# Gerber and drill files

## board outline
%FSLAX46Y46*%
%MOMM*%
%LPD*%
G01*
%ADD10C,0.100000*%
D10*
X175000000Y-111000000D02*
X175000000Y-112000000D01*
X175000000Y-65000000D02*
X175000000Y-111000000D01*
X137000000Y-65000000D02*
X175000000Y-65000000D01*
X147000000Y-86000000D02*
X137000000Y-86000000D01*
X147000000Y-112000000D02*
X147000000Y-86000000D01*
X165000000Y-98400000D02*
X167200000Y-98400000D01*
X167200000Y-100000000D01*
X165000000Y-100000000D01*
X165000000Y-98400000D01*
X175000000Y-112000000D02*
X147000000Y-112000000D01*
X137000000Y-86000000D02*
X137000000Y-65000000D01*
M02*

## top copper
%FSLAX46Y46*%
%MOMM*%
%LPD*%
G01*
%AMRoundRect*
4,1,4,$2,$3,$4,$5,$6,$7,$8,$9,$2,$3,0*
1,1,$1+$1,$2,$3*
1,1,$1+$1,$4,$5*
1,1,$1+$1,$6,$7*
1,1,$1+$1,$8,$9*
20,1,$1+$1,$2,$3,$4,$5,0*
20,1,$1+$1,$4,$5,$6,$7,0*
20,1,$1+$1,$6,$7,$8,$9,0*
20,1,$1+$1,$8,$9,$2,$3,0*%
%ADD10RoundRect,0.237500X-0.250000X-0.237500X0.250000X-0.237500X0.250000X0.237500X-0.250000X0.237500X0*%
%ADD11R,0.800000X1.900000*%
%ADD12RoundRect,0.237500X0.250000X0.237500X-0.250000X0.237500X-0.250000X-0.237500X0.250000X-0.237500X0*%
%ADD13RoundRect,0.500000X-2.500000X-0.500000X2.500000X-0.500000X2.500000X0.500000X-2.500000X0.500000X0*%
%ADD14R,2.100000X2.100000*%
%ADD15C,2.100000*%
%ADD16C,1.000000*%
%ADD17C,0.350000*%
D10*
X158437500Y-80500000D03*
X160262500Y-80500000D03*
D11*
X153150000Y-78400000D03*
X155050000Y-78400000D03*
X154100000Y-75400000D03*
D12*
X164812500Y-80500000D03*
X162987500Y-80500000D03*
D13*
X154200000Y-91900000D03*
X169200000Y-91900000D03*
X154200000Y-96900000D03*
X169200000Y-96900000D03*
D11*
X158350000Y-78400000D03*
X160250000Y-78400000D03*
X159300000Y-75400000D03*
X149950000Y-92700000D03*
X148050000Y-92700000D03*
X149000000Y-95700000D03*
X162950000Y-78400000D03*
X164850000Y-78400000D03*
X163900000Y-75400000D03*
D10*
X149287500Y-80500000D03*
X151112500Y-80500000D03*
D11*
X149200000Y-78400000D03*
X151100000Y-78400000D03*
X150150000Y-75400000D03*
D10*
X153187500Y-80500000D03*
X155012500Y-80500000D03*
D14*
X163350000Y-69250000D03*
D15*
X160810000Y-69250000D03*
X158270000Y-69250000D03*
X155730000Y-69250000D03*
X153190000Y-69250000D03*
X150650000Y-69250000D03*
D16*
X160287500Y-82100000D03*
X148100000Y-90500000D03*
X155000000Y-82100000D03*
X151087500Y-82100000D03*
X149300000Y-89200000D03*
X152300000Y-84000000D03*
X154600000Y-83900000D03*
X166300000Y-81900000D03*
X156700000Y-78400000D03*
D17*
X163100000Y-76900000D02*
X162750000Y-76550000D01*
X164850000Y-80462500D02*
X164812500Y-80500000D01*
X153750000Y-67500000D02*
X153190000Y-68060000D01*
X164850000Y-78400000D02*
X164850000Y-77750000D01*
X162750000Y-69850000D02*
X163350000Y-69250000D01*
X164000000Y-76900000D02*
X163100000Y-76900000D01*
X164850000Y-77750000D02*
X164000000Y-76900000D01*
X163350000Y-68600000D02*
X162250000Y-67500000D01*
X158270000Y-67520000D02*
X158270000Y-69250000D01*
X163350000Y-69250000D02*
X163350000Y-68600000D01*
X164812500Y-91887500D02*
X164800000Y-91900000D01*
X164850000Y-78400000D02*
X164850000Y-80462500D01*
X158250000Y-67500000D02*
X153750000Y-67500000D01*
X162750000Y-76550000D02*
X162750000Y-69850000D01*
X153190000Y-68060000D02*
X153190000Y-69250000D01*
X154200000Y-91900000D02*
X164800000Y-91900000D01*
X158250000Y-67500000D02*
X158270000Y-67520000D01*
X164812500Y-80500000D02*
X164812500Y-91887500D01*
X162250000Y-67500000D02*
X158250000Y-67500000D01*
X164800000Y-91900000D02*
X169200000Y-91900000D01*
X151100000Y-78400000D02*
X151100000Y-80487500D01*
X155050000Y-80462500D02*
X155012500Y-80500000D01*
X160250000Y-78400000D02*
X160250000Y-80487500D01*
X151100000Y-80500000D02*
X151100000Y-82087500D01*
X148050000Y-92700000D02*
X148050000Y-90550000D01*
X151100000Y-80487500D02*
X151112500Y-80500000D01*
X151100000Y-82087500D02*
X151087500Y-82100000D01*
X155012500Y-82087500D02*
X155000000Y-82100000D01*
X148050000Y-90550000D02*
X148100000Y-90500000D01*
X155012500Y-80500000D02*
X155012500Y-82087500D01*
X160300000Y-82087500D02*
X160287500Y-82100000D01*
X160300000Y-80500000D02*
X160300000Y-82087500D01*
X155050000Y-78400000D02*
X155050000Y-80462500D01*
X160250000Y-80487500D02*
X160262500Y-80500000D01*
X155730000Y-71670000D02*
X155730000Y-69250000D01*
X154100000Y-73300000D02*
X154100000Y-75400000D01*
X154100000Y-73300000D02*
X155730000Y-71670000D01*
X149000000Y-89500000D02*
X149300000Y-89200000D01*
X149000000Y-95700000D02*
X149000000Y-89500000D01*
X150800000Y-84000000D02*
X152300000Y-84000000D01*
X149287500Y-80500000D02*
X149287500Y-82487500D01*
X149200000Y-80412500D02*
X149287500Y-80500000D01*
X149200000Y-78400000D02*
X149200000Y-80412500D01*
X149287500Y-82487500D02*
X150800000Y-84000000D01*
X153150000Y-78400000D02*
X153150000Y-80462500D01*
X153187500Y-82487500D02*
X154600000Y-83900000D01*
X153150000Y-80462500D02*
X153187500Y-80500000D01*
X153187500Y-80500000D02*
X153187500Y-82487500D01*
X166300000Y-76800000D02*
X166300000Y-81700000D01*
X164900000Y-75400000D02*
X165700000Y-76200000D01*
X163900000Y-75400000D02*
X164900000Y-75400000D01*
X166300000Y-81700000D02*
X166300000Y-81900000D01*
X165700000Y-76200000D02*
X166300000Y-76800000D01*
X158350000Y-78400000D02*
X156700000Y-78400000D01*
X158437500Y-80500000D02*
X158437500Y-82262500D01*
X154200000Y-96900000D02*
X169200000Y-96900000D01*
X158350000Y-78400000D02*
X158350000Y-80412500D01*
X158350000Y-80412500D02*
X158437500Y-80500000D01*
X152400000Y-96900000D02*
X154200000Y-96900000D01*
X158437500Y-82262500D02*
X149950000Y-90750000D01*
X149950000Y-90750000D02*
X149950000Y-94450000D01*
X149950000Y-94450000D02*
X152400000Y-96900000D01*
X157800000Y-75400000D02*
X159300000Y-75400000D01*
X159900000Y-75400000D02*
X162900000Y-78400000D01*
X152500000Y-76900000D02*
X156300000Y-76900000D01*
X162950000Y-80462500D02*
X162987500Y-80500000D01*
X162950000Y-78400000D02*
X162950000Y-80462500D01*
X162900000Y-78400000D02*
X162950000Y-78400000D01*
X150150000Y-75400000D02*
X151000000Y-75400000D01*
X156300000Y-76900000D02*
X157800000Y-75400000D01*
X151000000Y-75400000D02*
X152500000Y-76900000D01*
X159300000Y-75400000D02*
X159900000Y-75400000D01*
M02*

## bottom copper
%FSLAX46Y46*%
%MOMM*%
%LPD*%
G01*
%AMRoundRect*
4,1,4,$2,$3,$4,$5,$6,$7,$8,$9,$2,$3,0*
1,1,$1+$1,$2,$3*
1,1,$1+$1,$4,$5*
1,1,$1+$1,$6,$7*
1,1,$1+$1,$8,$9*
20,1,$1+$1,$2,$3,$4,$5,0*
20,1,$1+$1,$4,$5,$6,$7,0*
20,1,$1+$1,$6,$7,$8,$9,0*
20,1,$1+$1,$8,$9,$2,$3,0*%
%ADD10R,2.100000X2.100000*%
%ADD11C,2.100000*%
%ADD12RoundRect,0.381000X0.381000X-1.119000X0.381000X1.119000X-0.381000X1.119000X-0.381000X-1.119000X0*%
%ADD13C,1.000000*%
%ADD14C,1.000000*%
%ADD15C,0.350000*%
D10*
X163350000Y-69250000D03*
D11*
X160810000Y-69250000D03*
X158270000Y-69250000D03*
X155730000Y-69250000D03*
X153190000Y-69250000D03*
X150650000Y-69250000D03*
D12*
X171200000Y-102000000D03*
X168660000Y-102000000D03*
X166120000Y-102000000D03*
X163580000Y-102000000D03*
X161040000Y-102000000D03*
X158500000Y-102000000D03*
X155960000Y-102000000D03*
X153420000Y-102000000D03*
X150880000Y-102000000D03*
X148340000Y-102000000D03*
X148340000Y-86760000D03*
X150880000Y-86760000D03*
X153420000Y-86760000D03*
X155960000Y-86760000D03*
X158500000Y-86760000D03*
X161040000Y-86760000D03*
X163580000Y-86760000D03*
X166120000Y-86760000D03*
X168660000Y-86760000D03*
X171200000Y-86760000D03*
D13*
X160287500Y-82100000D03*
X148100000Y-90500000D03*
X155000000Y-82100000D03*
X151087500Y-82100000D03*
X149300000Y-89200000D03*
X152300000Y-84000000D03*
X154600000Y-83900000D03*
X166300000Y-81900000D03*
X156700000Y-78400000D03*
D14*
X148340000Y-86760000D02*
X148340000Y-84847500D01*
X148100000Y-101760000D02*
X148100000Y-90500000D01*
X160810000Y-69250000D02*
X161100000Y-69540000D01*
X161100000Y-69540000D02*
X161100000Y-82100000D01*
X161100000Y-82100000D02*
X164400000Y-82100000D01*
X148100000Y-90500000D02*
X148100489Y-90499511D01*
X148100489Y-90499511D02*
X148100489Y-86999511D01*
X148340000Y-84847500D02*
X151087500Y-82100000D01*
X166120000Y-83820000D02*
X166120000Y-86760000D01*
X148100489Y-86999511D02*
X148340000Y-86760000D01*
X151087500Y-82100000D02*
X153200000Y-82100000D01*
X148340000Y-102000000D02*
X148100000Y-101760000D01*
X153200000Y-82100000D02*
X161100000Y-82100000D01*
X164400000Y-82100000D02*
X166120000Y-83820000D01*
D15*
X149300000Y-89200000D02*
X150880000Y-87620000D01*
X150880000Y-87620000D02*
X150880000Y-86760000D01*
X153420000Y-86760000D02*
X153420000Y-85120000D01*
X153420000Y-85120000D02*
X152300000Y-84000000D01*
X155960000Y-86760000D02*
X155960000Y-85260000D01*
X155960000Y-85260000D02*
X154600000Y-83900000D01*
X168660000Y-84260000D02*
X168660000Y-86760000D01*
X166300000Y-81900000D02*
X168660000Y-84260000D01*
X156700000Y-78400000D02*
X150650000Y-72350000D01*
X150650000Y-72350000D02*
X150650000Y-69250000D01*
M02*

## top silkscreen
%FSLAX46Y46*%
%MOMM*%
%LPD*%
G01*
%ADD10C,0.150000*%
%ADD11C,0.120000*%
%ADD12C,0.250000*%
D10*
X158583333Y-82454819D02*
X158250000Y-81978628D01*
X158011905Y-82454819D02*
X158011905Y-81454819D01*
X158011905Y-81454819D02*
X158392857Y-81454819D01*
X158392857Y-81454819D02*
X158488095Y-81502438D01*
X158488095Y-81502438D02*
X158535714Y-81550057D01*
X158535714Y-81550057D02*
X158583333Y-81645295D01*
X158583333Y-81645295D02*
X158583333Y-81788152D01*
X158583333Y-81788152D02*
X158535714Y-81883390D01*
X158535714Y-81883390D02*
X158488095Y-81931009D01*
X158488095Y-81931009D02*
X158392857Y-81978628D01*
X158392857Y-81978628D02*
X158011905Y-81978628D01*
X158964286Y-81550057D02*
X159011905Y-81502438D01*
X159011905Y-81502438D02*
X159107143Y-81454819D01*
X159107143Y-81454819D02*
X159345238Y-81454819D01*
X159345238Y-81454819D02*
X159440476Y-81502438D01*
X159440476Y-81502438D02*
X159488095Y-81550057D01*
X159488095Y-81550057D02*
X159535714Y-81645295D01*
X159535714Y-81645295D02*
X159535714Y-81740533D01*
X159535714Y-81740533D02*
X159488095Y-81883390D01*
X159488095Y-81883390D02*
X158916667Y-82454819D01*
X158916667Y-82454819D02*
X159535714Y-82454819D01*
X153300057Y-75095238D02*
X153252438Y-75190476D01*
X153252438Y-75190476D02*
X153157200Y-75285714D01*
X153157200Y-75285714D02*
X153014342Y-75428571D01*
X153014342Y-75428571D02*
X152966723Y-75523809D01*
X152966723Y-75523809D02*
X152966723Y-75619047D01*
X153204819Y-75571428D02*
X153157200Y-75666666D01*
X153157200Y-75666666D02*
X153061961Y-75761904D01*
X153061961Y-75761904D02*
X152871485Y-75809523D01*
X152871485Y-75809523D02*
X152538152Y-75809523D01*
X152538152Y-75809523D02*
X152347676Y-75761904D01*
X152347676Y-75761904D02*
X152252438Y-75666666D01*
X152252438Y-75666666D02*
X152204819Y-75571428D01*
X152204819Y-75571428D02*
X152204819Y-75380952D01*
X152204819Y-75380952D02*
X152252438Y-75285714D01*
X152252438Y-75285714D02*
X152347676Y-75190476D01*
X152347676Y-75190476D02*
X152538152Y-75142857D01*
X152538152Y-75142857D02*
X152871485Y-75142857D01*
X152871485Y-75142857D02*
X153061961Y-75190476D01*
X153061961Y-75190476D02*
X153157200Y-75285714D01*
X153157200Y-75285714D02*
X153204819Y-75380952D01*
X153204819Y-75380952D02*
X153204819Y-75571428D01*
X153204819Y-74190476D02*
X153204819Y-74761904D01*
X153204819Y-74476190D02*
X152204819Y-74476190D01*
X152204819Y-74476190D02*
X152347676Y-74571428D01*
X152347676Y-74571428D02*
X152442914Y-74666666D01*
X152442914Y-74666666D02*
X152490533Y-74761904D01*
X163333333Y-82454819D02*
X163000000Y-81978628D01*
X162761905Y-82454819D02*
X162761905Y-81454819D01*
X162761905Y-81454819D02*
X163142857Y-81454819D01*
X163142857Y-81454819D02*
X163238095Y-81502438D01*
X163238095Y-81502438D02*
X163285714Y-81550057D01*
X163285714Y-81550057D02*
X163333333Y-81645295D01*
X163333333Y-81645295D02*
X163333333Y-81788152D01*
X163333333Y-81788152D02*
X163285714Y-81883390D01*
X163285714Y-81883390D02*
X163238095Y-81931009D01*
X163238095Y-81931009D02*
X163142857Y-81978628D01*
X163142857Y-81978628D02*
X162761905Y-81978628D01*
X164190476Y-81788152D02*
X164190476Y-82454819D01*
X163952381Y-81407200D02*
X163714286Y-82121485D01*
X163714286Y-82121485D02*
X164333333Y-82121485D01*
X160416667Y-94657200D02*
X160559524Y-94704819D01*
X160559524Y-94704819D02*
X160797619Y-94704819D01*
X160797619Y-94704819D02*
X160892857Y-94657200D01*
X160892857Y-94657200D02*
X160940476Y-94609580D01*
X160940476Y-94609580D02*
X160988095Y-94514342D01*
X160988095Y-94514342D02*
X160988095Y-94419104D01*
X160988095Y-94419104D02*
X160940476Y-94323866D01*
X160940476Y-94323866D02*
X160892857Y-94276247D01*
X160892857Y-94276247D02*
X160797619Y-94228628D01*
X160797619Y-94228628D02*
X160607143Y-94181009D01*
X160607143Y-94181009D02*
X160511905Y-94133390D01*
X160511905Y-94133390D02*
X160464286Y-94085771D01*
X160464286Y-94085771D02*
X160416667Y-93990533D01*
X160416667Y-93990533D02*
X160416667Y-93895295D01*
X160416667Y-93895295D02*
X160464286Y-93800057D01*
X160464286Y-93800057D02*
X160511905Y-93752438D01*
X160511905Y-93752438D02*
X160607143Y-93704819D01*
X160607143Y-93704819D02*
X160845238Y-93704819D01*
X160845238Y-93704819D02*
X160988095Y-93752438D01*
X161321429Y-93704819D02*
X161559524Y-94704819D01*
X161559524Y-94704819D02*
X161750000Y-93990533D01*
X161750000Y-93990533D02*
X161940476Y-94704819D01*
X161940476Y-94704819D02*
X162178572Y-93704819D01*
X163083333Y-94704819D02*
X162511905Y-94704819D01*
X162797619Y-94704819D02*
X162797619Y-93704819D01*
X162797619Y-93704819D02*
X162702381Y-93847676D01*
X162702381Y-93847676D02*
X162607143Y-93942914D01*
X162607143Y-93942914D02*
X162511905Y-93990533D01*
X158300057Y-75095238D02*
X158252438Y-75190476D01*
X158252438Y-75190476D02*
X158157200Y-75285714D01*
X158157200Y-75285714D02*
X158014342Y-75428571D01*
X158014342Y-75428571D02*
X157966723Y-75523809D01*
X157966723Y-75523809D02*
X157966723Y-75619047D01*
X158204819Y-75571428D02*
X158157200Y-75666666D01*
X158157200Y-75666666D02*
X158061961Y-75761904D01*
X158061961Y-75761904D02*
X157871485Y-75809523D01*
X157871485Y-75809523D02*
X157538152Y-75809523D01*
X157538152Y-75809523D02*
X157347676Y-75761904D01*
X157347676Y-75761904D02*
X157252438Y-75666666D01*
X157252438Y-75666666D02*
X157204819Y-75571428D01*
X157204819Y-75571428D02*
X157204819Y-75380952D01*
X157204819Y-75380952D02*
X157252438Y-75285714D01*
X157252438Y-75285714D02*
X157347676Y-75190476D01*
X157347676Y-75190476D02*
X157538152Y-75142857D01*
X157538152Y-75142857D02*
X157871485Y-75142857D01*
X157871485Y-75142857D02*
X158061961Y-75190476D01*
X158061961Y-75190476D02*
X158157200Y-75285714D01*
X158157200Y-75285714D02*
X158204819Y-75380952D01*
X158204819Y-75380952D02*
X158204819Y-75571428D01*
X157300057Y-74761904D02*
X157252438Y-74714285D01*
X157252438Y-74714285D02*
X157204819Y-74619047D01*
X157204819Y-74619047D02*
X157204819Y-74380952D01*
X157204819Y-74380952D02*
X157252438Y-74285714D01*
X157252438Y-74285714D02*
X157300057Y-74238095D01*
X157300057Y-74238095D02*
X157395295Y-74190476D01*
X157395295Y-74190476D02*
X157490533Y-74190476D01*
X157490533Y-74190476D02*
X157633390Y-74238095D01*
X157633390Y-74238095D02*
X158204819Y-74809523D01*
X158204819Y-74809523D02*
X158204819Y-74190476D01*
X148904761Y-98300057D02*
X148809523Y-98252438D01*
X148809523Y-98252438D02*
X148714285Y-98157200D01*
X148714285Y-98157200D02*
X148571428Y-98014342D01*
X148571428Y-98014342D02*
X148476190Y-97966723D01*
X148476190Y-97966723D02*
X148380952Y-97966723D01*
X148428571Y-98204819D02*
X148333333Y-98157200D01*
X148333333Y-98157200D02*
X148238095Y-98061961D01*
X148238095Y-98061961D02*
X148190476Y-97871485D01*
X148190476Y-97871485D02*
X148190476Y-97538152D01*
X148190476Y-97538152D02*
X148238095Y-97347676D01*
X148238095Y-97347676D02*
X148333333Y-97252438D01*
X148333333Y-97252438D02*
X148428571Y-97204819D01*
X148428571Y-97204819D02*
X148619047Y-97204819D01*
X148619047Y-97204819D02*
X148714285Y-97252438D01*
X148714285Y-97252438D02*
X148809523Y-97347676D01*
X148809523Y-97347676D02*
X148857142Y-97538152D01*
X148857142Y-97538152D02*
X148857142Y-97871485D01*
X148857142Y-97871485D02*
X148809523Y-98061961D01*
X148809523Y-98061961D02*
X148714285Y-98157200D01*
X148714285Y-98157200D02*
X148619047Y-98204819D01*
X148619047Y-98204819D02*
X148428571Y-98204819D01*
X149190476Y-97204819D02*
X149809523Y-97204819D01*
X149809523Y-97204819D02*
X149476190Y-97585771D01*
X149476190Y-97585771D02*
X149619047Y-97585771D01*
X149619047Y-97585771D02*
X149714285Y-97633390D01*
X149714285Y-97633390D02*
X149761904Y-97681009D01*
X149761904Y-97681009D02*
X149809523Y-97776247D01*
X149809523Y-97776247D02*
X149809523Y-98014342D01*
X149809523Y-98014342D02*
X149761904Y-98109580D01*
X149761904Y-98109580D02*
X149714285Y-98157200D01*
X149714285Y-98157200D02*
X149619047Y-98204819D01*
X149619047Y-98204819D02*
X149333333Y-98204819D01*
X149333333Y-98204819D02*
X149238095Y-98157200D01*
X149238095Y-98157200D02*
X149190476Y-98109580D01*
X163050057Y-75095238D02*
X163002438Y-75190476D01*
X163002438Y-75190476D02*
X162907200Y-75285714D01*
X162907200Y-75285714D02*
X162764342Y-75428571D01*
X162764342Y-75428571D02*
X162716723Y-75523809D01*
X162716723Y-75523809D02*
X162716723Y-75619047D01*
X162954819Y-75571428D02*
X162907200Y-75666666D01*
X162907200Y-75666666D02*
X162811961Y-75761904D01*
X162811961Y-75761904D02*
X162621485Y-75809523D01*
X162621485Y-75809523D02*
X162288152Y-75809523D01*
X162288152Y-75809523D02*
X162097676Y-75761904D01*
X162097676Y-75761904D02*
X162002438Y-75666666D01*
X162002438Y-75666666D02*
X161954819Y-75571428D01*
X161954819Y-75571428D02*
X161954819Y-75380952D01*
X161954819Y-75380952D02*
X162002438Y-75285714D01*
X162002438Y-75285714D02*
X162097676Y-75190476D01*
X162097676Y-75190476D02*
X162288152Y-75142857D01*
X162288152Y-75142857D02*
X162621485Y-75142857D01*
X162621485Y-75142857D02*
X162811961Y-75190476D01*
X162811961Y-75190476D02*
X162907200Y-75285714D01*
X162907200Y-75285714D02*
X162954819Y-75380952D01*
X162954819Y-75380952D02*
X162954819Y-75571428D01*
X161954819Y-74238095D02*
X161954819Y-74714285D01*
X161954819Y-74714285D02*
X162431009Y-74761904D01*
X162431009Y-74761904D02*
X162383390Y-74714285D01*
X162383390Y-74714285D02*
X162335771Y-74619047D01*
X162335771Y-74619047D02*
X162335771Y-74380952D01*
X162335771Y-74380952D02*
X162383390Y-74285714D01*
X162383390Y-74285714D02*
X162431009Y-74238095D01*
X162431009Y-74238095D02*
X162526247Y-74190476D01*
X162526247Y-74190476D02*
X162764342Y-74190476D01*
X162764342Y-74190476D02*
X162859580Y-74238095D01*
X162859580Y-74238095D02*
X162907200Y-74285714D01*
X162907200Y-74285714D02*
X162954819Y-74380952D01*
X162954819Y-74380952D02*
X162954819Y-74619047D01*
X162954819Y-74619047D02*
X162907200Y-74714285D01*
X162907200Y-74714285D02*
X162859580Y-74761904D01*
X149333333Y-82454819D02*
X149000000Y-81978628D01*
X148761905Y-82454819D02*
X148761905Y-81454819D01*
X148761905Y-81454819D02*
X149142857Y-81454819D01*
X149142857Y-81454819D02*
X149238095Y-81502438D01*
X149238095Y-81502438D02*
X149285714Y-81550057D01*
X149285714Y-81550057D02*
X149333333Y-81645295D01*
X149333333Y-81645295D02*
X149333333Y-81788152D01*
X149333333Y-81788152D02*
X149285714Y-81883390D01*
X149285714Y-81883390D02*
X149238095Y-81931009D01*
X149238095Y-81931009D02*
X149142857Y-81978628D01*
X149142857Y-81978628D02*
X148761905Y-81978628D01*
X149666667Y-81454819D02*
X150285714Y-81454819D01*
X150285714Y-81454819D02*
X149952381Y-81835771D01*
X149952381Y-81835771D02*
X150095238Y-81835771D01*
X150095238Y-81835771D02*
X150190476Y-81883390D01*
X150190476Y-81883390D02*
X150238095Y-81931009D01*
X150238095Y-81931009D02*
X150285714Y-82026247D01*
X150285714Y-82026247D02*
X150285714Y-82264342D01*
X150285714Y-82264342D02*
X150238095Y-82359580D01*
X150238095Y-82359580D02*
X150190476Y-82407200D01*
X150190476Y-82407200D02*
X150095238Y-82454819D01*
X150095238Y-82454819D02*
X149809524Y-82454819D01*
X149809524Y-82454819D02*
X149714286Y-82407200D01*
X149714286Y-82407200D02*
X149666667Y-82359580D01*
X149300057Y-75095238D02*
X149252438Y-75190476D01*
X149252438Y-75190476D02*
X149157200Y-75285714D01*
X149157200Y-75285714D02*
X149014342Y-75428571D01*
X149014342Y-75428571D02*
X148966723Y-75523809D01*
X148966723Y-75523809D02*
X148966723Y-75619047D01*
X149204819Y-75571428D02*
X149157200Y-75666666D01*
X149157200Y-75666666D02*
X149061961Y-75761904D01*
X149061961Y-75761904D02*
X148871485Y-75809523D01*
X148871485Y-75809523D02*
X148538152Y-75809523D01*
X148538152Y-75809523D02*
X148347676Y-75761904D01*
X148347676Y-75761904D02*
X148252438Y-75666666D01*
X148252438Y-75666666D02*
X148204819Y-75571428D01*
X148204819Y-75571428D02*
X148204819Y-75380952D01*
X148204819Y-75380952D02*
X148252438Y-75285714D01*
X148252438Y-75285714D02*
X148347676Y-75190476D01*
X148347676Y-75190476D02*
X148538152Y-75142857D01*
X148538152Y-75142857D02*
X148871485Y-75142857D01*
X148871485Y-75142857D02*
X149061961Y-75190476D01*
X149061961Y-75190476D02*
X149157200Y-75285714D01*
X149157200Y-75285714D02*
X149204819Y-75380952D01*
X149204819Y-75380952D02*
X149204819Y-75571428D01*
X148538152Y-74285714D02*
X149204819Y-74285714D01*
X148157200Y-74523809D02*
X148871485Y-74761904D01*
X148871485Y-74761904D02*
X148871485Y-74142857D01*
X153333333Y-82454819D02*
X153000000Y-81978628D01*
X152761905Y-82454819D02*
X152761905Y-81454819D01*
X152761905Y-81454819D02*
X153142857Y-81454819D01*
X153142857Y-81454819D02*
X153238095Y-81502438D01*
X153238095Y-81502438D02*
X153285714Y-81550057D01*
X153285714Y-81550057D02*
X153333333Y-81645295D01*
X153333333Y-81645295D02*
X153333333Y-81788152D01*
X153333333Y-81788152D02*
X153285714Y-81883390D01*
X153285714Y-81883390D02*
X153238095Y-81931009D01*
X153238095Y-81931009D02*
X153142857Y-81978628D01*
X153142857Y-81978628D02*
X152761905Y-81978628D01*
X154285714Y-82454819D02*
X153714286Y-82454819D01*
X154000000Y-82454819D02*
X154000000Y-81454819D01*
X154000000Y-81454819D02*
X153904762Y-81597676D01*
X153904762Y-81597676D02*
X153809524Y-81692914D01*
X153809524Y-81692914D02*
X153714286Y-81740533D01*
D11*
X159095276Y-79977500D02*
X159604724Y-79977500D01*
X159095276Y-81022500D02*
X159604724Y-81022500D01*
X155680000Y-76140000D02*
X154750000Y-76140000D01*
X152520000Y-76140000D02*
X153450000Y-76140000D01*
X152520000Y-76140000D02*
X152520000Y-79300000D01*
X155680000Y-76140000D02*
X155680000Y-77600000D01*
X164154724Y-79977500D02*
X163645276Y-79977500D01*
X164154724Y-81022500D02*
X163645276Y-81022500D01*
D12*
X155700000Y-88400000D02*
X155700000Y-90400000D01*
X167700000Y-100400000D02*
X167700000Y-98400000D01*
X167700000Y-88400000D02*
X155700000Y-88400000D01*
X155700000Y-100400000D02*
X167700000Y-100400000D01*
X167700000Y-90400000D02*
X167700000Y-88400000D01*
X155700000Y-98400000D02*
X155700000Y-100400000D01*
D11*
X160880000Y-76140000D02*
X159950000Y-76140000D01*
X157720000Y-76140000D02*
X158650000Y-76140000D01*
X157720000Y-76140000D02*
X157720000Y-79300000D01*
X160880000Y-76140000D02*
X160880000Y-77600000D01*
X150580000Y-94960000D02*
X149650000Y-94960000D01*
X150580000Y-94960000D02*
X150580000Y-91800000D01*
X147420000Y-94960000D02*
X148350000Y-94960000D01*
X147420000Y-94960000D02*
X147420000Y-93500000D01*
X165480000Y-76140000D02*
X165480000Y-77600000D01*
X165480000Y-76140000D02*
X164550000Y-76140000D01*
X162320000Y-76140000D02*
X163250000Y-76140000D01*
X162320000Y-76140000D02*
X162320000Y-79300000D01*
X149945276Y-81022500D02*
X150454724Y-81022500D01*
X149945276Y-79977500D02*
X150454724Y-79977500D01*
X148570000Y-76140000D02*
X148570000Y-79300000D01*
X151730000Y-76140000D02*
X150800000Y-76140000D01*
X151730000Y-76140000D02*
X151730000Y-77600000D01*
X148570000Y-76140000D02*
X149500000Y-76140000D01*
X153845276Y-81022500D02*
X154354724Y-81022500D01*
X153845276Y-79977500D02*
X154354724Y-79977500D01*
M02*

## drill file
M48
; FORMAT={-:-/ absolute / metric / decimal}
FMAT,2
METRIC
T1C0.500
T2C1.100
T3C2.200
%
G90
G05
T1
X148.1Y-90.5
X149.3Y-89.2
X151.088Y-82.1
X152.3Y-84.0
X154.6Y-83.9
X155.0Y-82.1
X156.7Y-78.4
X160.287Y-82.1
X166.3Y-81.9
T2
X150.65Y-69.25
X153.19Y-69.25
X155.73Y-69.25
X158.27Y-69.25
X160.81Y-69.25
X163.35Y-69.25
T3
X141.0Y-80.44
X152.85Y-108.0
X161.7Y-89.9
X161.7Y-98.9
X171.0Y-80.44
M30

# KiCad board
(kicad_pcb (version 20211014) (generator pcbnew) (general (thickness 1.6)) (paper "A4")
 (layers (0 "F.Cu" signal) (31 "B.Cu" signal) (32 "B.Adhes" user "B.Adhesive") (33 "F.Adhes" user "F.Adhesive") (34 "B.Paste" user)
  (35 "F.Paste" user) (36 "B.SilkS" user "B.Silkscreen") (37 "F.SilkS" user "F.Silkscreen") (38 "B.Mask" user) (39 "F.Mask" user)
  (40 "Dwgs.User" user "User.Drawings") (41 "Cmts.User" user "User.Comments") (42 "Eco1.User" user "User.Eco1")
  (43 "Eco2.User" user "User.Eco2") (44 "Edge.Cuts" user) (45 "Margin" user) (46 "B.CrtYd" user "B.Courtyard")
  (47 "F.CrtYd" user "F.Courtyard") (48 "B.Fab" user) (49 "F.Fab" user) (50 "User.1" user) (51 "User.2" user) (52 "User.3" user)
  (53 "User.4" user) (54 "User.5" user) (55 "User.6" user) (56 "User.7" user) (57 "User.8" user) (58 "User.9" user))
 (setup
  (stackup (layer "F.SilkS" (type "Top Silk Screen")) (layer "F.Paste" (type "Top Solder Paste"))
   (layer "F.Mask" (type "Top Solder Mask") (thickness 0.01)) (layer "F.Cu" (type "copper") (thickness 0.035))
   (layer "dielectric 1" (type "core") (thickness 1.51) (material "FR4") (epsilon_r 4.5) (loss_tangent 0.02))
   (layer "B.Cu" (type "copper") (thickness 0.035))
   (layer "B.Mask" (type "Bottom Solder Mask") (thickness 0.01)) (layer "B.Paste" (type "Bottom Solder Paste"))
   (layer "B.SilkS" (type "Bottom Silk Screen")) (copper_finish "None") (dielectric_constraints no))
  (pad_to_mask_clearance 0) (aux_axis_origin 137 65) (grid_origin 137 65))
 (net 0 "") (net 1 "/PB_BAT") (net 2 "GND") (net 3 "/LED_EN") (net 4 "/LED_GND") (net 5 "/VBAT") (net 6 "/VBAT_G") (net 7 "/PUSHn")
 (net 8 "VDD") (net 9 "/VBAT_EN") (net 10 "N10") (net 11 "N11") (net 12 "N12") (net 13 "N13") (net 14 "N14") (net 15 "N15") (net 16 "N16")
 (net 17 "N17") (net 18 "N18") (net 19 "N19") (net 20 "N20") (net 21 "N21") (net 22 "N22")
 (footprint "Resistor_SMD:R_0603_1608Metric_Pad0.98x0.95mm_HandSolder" (layer "F.Cu") (at 159.35 80.5)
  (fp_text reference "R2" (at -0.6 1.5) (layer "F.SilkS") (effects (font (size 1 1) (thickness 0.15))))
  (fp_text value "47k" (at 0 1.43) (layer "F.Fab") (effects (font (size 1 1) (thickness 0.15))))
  (fp_line (start -0.254724 -0.5225) (end 0.254724 -0.5225) (layer "F.SilkS") (width 0.12))
  (fp_line (start -0.254724 0.5225) (end 0.254724 0.5225) (layer "F.SilkS") (width 0.12))
  (pad "1" smd roundrect (at -0.9125 0) (size 0.975 0.95) (layers "F.Cu" "F.Paste" "F.Mask") (roundrect_rratio 0.25) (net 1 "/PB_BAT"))
  (pad "2" smd roundrect (at 0.9125 0) (size 0.975 0.95) (layers "F.Cu" "F.Paste" "F.Mask") (roundrect_rratio 0.25) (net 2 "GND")))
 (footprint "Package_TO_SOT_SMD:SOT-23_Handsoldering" (layer "F.Cu") (at 154.1 76.9 90)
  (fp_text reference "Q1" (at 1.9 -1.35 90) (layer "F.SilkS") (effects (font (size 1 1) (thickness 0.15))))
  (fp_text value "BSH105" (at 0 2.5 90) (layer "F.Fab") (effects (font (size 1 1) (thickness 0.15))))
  (fp_line (start 0.76 1.58) (end 0.76 0.65) (layer "F.SilkS") (width 0.12))
  (fp_line (start 0.76 -1.58) (end 0.76 -0.65) (layer "F.SilkS") (width 0.12))
  (fp_line (start 0.76 -1.58) (end -2.4 -1.58) (layer "F.SilkS") (width 0.12))
  (fp_line (start 0.76 1.58) (end -0.7 1.58) (layer "F.SilkS") (width 0.12))
  (pad "1" smd rect (at -1.5 -0.95 90) (size 1.9 0.8) (layers "F.Cu" "F.Paste" "F.Mask") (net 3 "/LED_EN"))
  (pad "2" smd rect (at -1.5 0.95 90) (size 1.9 0.8) (layers "F.Cu" "F.Paste" "F.Mask") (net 2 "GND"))
  (pad "3" smd rect (at 1.5 0 90) (size 1.9 0.8) (layers "F.Cu" "F.Paste" "F.Mask") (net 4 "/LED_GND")))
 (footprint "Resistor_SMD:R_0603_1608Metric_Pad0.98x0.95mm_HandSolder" (layer "F.Cu") (at 163.9 80.5 180)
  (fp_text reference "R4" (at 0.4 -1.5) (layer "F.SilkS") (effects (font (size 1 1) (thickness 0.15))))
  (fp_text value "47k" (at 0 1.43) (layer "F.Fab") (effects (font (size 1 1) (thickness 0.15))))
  (fp_line (start -0.254724 0.5225) (end 0.254724 0.5225) (layer "F.SilkS") (width 0.12))
  (fp_line (start -0.254724 -0.5225) (end 0.254724 -0.5225) (layer "F.SilkS") (width 0.12))
  (pad "1" smd roundrect (at -0.9125 0 180) (size 0.975 0.95) (layers "F.Cu" "F.Paste" "F.Mask") (roundrect_rratio 0.25) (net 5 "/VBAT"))
  (pad "2" smd roundrect (at 0.9125 0 180) (size 0.975 0.95) (layers "F.Cu" "F.Paste" "F.Mask") (roundrect_rratio 0.25) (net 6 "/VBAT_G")))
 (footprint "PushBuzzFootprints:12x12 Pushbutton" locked (layer "F.Cu") (at 154.2 91.9)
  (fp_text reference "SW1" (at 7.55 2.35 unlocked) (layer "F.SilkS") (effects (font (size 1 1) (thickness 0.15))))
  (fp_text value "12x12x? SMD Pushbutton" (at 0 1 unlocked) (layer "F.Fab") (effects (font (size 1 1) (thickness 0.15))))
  (fp_line (start 1.5 -3.5) (end 1.5 -1.5) (layer "F.SilkS") (width 0.25))
  (fp_line (start 13.5 8.5) (end 13.5 6.5) (layer "F.SilkS") (width 0.25))
  (fp_line (start 13.5 -3.5) (end 1.5 -3.5) (layer "F.SilkS") (width 0.25))
  (fp_line (start 1.5 8.5) (end 13.5 8.5) (layer "F.SilkS") (width 0.25))
  (fp_line (start 13.5 -1.5) (end 13.5 -3.5) (layer "F.SilkS") (width 0.25))
  (fp_line (start 1.5 6.5) (end 1.5 8.5) (layer "F.SilkS") (width 0.25))
  (pad "" np_thru_hole circle locked (at 7.5 -2) (size 2 2) (drill 2.2) (layers F&B.Cu *.Mask))
  (pad "" np_thru_hole circle locked (at 7.5 7) (size 2 2) (drill 2.2) (layers F&B.Cu *.Mask))
  (pad "1" smd roundrect locked (at 0 0) (size 6 2) (layers "F.Cu" "F.Paste" "F.Mask") (roundrect_rratio 0.25) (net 5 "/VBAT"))
  (pad "1" smd roundrect locked (at 15 0) (size 6 2) (layers "F.Cu" "F.Paste" "F.Mask") (roundrect_rratio 0.25) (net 5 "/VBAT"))
  (pad "2" smd roundrect locked (at 0 5) (size 6 2) (layers "F.Cu" "F.Paste" "F.Mask") (roundrect_rratio 0.25) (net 1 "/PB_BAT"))
  (pad "2" smd roundrect locked (at 15 5) (size 6 2) (layers "F.Cu" "F.Paste" "F.Mask") (roundrect_rratio 0.25) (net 1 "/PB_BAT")))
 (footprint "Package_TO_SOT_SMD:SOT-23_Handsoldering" (layer "F.Cu") (at 159.3 76.9 90)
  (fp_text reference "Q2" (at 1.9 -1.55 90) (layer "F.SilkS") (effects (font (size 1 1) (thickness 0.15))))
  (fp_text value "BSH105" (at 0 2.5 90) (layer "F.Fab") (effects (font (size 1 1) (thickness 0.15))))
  (fp_line (start 0.76 1.58) (end 0.76 0.65) (layer "F.SilkS") (width 0.12))
  (fp_line (start 0.76 -1.58) (end 0.76 -0.65) (layer "F.SilkS") (width 0.12))
  (fp_line (start 0.76 -1.58) (end -2.4 -1.58) (layer "F.SilkS") (width 0.12))
  (fp_line (start 0.76 1.58) (end -0.7 1.58) (layer "F.SilkS") (width 0.12))
  (pad "1" smd rect (at -1.5 -0.95 90) (size 1.9 0.8) (layers "F.Cu" "F.Paste" "F.Mask") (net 1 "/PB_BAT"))
  (pad "2" smd rect (at -1.5 0.95 90) (size 1.9 0.8) (layers "F.Cu" "F.Paste" "F.Mask") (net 2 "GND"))
  (pad "3" smd rect (at 1.5 0 90) (size 1.9 0.8) (layers "F.Cu" "F.Paste" "F.Mask") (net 6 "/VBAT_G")))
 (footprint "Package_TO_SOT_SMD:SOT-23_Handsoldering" (layer "F.Cu") (at 149 94.2 -90)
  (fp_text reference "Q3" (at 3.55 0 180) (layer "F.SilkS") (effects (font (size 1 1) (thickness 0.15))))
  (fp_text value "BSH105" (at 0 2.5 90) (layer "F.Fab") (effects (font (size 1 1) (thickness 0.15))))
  (fp_line (start 0.76 -1.58) (end 0.76 -0.65) (layer "F.SilkS") (width 0.12))
  (fp_line (start 0.76 -1.58) (end -2.4 -1.58) (layer "F.SilkS") (width 0.12))
  (fp_line (start 0.76 1.58) (end 0.76 0.65) (layer "F.SilkS") (width 0.12))
  (fp_line (start 0.76 1.58) (end -0.7 1.58) (layer "F.SilkS") (width 0.12))
  (pad "1" smd rect (at -1.5 -0.95 270) (size 1.9 0.8) (layers "F.Cu" "F.Paste" "F.Mask") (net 1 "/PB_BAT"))
  (pad "2" smd rect (at -1.5 0.95 270) (size 1.9 0.8) (layers "F.Cu" "F.Paste" "F.Mask") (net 2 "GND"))
  (pad "3" smd rect (at 1.5 0 270) (size 1.9 0.8) (layers "F.Cu" "F.Paste" "F.Mask") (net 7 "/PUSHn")))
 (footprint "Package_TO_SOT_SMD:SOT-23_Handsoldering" (layer "F.Cu") (at 163.9 76.9 90)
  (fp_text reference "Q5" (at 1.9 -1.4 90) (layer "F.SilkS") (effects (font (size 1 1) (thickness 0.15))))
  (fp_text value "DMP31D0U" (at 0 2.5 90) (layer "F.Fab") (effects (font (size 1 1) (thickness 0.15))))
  (fp_line (start 0.76 1.58) (end -0.7 1.58) (layer "F.SilkS") (width 0.12))
  (fp_line (start 0.76 1.58) (end 0.76 0.65) (layer "F.SilkS") (width 0.12))
  (fp_line (start 0.76 -1.58) (end 0.76 -0.65) (layer "F.SilkS") (width 0.12))
  (fp_line (start 0.76 -1.58) (end -2.4 -1.58) (layer "F.SilkS") (width 0.12))
  (pad "1" smd rect (at -1.5 -0.95 90) (size 1.9 0.8) (layers "F.Cu" "F.Paste" "F.Mask") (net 6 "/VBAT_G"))
  (pad "2" smd rect (at -1.5 0.95 90) (size 1.9 0.8) (layers "F.Cu" "F.Paste" "F.Mask") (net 5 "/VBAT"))
  (pad "3" smd rect (at 1.5 0 90) (size 1.9 0.8) (layers "F.Cu" "F.Paste" "F.Mask") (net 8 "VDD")))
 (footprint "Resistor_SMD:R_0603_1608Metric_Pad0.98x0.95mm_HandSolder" (layer "F.Cu") (at 150.2 80.5)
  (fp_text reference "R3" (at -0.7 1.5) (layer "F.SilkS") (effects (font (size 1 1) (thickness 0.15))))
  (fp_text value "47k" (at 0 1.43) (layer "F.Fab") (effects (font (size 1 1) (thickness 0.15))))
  (fp_line (start -0.254724 0.5225) (end 0.254724 0.5225) (layer "F.SilkS") (width 0.12))
  (fp_line (start -0.254724 -0.5225) (end 0.254724 -0.5225) (layer "F.SilkS") (width 0.12))
  (pad "1" smd roundrect (at -0.9125 0) (size 0.975 0.95) (layers "F.Cu" "F.Paste" "F.Mask") (roundrect_rratio 0.25) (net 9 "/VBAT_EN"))
  (pad "2" smd roundrect (at 0.9125 0) (size 0.975 0.95) (layers "F.Cu" "F.Paste" "F.Mask") (roundrect_rratio 0.25) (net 2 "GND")))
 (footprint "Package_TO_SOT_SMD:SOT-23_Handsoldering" (layer "F.Cu") (at 150.15 76.9 90)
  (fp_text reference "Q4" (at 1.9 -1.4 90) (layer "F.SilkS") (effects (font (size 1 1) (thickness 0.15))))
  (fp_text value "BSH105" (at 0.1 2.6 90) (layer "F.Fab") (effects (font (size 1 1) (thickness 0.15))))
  (fp_line (start 0.76 -1.58) (end -2.4 -1.58) (layer "F.SilkS") (width 0.12))
  (fp_line (start 0.76 1.58) (end 0.76 0.65) (layer "F.SilkS") (width 0.12))
  (fp_line (start 0.76 1.58) (end -0.7 1.58) (layer "F.SilkS") (width 0.12))
  (fp_line (start 0.76 -1.58) (end 0.76 -0.65) (layer "F.SilkS") (width 0.12))
  (pad "1" smd rect (at -1.5 -0.95 90) (size 1.9 0.8) (layers "F.Cu" "F.Paste" "F.Mask") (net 9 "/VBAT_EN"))
  (pad "2" smd rect (at -1.5 0.95 90) (size 1.9 0.8) (layers "F.Cu" "F.Paste" "F.Mask") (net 2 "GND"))
  (pad "3" smd rect (at 1.5 0 90) (size 1.9 0.8) (layers "F.Cu" "F.Paste" "F.Mask") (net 6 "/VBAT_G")))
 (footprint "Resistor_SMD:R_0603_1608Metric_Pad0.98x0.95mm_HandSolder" (layer "F.Cu") (at 154.1 80.5)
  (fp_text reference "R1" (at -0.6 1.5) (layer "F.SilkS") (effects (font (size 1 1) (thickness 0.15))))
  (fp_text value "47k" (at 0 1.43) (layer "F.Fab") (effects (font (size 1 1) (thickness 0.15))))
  (fp_line (start -0.254724 0.5225) (end 0.254724 0.5225) (layer "F.SilkS") (width 0.12))
  (fp_line (start -0.254724 -0.5225) (end 0.254724 -0.5225) (layer "F.SilkS") (width 0.12))
  (pad "1" smd roundrect (at -0.9125 0) (size 0.975 0.95) (layers "F.Cu" "F.Paste" "F.Mask") (roundrect_rratio 0.25) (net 3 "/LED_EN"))
  (pad "2" smd roundrect (at 0.9125 0) (size 0.975 0.95) (layers "F.Cu" "F.Paste" "F.Mask") (roundrect_rratio 0.25) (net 2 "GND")))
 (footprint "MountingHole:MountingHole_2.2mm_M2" (layer "B.Cu") (at 152.85 108 180)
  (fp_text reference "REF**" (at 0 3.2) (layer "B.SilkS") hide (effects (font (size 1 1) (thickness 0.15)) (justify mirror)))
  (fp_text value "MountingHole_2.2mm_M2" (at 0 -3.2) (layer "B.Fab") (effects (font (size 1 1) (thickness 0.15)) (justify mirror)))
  (pad "" np_thru_hole circle (at 0 0 180) (size 2.2 2.2) (drill 2.2) (layers *.Cu *.Mask)))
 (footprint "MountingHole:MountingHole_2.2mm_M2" (layer "B.Cu") (at 141 80.44 180)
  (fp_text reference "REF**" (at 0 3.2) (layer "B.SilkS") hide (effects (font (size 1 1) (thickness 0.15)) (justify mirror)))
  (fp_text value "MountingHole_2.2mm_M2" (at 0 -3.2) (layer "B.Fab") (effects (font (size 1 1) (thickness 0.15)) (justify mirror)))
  (pad "" np_thru_hole circle (at 0 0 180) (size 2.2 2.2) (drill 2.2) (layers *.Cu *.Mask)))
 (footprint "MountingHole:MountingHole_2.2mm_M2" (layer "B.Cu") (at 171 80.44 180)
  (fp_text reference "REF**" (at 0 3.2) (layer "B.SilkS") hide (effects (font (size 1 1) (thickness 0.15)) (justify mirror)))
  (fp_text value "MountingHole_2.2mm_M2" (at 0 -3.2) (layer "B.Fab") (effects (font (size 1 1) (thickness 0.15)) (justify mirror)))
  (pad "" np_thru_hole circle (at 0 0 180) (size 2.2 2.2) (drill 2.2) (layers *.Cu *.Mask)))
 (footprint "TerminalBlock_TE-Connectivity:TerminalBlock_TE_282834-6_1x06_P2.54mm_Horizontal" (layer "B.Cu") (at 163.35 69.25 180)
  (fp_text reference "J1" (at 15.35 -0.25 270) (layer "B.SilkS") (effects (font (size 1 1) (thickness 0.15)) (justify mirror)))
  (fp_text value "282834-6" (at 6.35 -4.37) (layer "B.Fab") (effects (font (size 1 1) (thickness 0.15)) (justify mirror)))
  (pad "1" thru_hole rect (at 0 0 180) (size 2.1 2.1) (drill 1.1) (layers *.Cu *.Mask) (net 5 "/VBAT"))
  (pad "2" thru_hole circle (at 2.54 0 180) (size 2.1 2.1) (drill 1.1) (layers *.Cu *.Mask) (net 2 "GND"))
  (pad "3" thru_hole circle (at 5.08 0 180) (size 2.1 2.1) (drill 1.1) (layers *.Cu *.Mask) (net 5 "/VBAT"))
  (pad "4" thru_hole circle (at 7.62 0 180) (size 2.1 2.1) (drill 1.1) (layers *.Cu *.Mask) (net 4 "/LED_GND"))
  (pad "5" thru_hole circle (at 10.16 0 180) (size 2.1 2.1) (drill 1.1) (layers *.Cu *.Mask) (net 5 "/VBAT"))
  (pad "6" thru_hole circle (at 12.7 0 180) (size 2.1 2.1) (drill 1.1) (layers *.Cu *.Mask) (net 1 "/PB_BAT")))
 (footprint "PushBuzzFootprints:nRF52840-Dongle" (layer "B.Cu") (at 171.2 102 90)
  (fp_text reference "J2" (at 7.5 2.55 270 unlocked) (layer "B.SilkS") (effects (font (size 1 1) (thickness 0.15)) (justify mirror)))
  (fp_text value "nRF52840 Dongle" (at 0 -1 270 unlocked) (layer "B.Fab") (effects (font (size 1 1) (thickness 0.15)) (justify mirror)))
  (pad "1" smd roundrect (at 0 0 90) (size 3 1.524) (layers "B.Cu" "B.Paste" "B.Mask") (roundrect_rratio 0.25) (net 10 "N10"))
  (pad "2" smd roundrect (at 0 -2.54 90) (size 3 1.524) (layers "B.Cu" "B.Paste" "B.Mask") (roundrect_rratio 0.25) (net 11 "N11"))
  (pad "3" smd roundrect (at 0 -5.08 90) (size 3 1.524) (layers "B.Cu" "B.Paste" "B.Mask") (roundrect_rratio 0.25) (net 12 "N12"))
  (pad "4" smd roundrect (at 0 -7.62 90) (size 3 1.524) (layers "B.Cu" "B.Paste" "B.Mask") (roundrect_rratio 0.25) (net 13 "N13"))
  (pad "5" smd roundrect (at 0 -10.16 90) (size 3 1.524) (layers "B.Cu" "B.Paste" "B.Mask") (roundrect_rratio 0.25) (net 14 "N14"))
  (pad "6" smd roundrect (at 0 -12.7 90) (size 3 1.524) (layers "B.Cu" "B.Paste" "B.Mask") (roundrect_rratio 0.25) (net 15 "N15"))
  (pad "7" smd roundrect (at 0 -15.24 90) (size 3 1.524) (layers "B.Cu" "B.Paste" "B.Mask") (roundrect_rratio 0.25) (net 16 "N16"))
  (pad "8" smd roundrect (at 0 -17.78 90) (size 3 1.524) (layers "B.Cu" "B.Paste" "B.Mask") (roundrect_rratio 0.25) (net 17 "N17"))
  (pad "9" smd roundrect (at 0 -20.32 90) (size 3 1.524) (layers "B.Cu" "B.Paste" "B.Mask") (roundrect_rratio 0.25) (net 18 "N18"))
  (pad "10" smd roundrect (at 0 -22.86 90) (size 3 1.524) (layers "B.Cu" "B.Paste" "B.Mask") (roundrect_rratio 0.25) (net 2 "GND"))
  (pad "11" smd roundrect (at 15.24 -22.86 90) (size 3 1.524) (layers "B.Cu" "B.Paste" "B.Mask") (roundrect_rratio 0.25) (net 2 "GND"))
  (pad "12" smd roundrect (at 15.24 -20.32 90) (size 3 1.524) (layers "B.Cu" "B.Paste" "B.Mask") (roundrect_rratio 0.25) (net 7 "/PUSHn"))
  (pad "13" smd roundrect (at 15.24 -17.78 90) (size 3 1.524) (layers "B.Cu" "B.Paste" "B.Mask") (roundrect_rratio 0.25) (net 9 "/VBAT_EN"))
  (pad "14" smd roundrect (at 15.24 -15.24 90) (size 3 1.524) (layers "B.Cu" "B.Paste" "B.Mask") (roundrect_rratio 0.25) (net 3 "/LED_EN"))
  (pad "15" smd roundrect (at 15.24 -12.7 90) (size 3 1.524) (layers "B.Cu" "B.Paste" "B.Mask") (roundrect_rratio 0.25) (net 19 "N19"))
  (pad "16" smd roundrect (at 15.24 -10.16 90) (size 3 1.524) (layers "B.Cu" "B.Paste" "B.Mask") (roundrect_rratio 0.25) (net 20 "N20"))
  (pad "17" smd roundrect (at 15.24 -7.62 90) (size 3 1.524) (layers "B.Cu" "B.Paste" "B.Mask") (roundrect_rratio 0.25) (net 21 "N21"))
  (pad "18" smd roundrect (at 15.24 -5.08 90) (size 3 1.524) (layers "B.Cu" "B.Paste" "B.Mask") (roundrect_rratio 0.25) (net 2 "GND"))
  (pad "19" smd roundrect (at 15.24 -2.54 90) (size 3 1.524) (layers "B.Cu" "B.Paste" "B.Mask") (roundrect_rratio 0.25) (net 8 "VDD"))
  (pad "20" smd roundrect (at 15.24 0 90) (size 3 1.524) (layers "B.Cu" "B.Paste" "B.Mask") (roundrect_rratio 0.25) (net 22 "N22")))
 (gr_line (start 175 111) (end 175 112) (layer "Edge.Cuts") (width 0.1))
 (gr_line (start 175 65) (end 175 111) (layer "Edge.Cuts") (width 0.1))
 (gr_line (start 137 65) (end 175 65) (layer "Edge.Cuts") (width 0.1))
 (gr_line (start 147 86) (end 137 86) (layer "Edge.Cuts") (width 0.1))
 (gr_line (start 147 112) (end 147 86) (layer "Edge.Cuts") (width 0.1))
 (gr_rect locked (start 165 100) (end 167.2 98.4) (layer "Edge.Cuts") (width 0.1) (fill none))
 (gr_line (start 175 112) (end 147 112) (layer "Edge.Cuts") (width 0.1))
 (gr_line (start 137 86) (end 137 65) (layer "Edge.Cuts") (width 0.1))
 (segment (start 163.1 76.9) (end 162.75 76.55) (width 0.35) (layer "F.Cu") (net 5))
 (segment (start 164.85 80.4625) (end 164.8125 80.5) (width 0.35) (layer "F.Cu") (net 5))
 (segment (start 153.75 67.5) (end 153.19 68.06) (width 0.35) (layer "F.Cu") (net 5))
 (segment (start 164.85 78.4) (end 164.85 77.75) (width 0.35) (layer "F.Cu") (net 5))
 (segment (start 162.75 69.85) (end 163.35 69.25) (width 0.35) (layer "F.Cu") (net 5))
 (segment (start 164 76.9) (end 163.1 76.9) (width 0.35) (layer "F.Cu") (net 5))
 (segment (start 164.85 77.75) (end 164 76.9) (width 0.35) (layer "F.Cu") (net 5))
 (segment (start 163.35 68.6) (end 162.25 67.5) (width 0.35) (layer "F.Cu") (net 5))
 (segment (start 158.27 67.52) (end 158.27 69.25) (width 0.35) (layer "F.Cu") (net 5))
 (segment (start 163.35 69.25) (end 163.35 68.6) (width 0.35) (layer "F.Cu") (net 5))
 (segment (start 164.8125 91.8875) (end 164.8 91.9) (width 0.35) (layer "F.Cu") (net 5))
 (segment (start 164.85 78.4) (end 164.85 80.4625) (width 0.35) (layer "F.Cu") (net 5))
 (segment (start 158.25 67.5) (end 153.75 67.5) (width 0.35) (layer "F.Cu") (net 5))
 (segment (start 162.75 76.55) (end 162.75 69.85) (width 0.35) (layer "F.Cu") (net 5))
 (segment (start 153.19 68.06) (end 153.19 69.25) (width 0.35) (layer "F.Cu") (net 5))
 (segment (start 154.2 91.9) (end 164.8 91.9) (width 0.35) (layer "F.Cu") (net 5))
 (segment (start 158.25 67.5) (end 158.27 67.52) (width 0.35) (layer "F.Cu") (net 5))
 (segment (start 164.8125 80.5) (end 164.8125 91.8875) (width 0.35) (layer "F.Cu") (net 5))
 (segment (start 162.25 67.5) (end 158.25 67.5) (width 0.35) (layer "F.Cu") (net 5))
 (segment (start 164.8 91.9) (end 169.2 91.9) (width 0.35) (layer "F.Cu") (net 5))
 (segment (start 151.1 78.4) (end 151.1 80.4875) (width 0.35) (layer "F.Cu") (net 2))
 (segment (start 155.05 80.4625) (end 155.0125 80.5) (width 0.35) (layer "F.Cu") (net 2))
 (segment (start 160.25 78.4) (end 160.25 80.4875) (width 0.35) (layer "F.Cu") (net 2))
 (segment (start 151.1 80.5) (end 151.1 82.0875) (width 0.35) (layer "F.Cu") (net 2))
 (segment (start 148.05 92.7) (end 148.05 90.55) (width 0.35) (layer "F.Cu") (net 2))
 (segment (start 151.1 80.4875) (end 151.1125 80.5) (width 0.35) (layer "F.Cu") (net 2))
 (segment (start 151.1 82.0875) (end 151.0875 82.1) (width 0.35) (layer "F.Cu") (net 2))
 (segment (start 155.0125 82.0875) (end 155 82.1) (width 0.35) (layer "F.Cu") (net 2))
 (segment (start 148.05 90.55) (end 148.1 90.5) (width 0.35) (layer "F.Cu") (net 2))
 (segment (start 155.0125 80.5) (end 155.0125 82.0875) (width 0.35) (layer "F.Cu") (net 2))
 (segment (start 160.3 82.0875) (end 160.2875 82.1) (width 0.35) (layer "F.Cu") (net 2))
 (segment (start 160.3 80.5) (end 160.3 82.0875) (width 0.35) (layer "F.Cu") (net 2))
 (segment (start 155.05 78.4) (end 155.05 80.4625) (width 0.35) (layer "F.Cu") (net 2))
 (segment (start 160.25 80.4875) (end 160.2625 80.5) (width 0.35) (layer "F.Cu") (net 2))
 (via (at 160.2875 82.1) (size 1) (drill 0.5) (layers "F.Cu" "B.Cu") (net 2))
 (via (at 148.1 90.5) (size 1) (drill 0.5) (layers "F.Cu" "B.Cu") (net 2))
 (via (at 155 82.1) (size 1) (drill 0.5) (layers "F.Cu" "B.Cu") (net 2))
 (via (at 151.0875 82.1) (size 1) (drill 0.5) (layers "F.Cu" "B.Cu") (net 2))
 (segment (start 148.34 86.76) (end 148.34 84.8475) (width 1) (layer "B.Cu") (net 2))
 (segment (start 148.1 101.76) (end 148.1 90.5) (width 1) (layer "B.Cu") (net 2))
 (segment (start 160.81 69.25) (end 161.1 69.54) (width 1) (layer "B.Cu") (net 2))
 (segment (start 161.1 69.54) (end 161.1 82.1) (width 1) (layer "B.Cu") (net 2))
 (segment (start 161.1 82.1) (end 164.4 82.1) (width 1) (layer "B.Cu") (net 2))
 (segment (start 148.1 90.5) (end 148.100489 90.499511) (width 1) (layer "B.Cu") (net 2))
 (segment (start 148.100489 90.499511) (end 148.100489 86.999511) (width 1) (layer "B.Cu") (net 2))
 (segment (start 148.34 84.8475) (end 151.0875 82.1) (width 1) (layer "B.Cu") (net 2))
 (segment (start 166.12 83.82) (end 166.12 86.76) (width 1) (layer "B.Cu") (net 2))
 (segment (start 148.100489 86.999511) (end 148.34 86.76) (width 1) (layer "B.Cu") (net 2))
 (segment (start 151.0875 82.1) (end 153.2 82.1) (width 1) (layer "B.Cu") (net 2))
 (segment (start 148.34 102) (end 148.1 101.76) (width 1) (layer "B.Cu") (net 2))
 (segment (start 153.2 82.1) (end 161.1 82.1) (width 1) (layer "B.Cu") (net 2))
 (segment (start 164.4 82.1) (end 166.12 83.82) (width 1) (layer "B.Cu") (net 2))
 (segment (start 155.73 71.67) (end 155.73 69.25) (width 0.35) (layer "F.Cu") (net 4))
 (segment (start 154.1 73.3) (end 154.1 75.4) (width 0.35) (layer "F.Cu") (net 4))
 (segment (start 154.1 73.3) (end 155.73 71.67) (width 0.35) (layer "F.Cu") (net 4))
 (segment (start 149 89.5) (end 149.3 89.2) (width 0.35) (layer "F.Cu") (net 7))
 (segment (start 149 95.7) (end 149 89.5) (width 0.35) (layer "F.Cu") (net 7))
 (via (at 149.3 89.2) (size 1) (drill 0.5) (layers "F.Cu" "B.Cu") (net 7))
 (segment (start 149.3 89.2) (end 150.88 87.62) (width 0.35) (layer "B.Cu") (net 7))
 (segment (start 150.88 87.62) (end 150.88 86.76) (width 0.35) (layer "B.Cu") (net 7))
 (segment (start 150.8 84) (end 152.3 84) (width 0.35) (layer "F.Cu") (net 9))
 (segment (start 149.2875 80.5) (end 149.2875 82.4875) (width 0.35) (layer "F.Cu") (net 9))
 (segment (start 149.2 80.4125) (end 149.2875 80.5) (width 0.35) (layer "F.Cu") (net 9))
 (segment (start 149.2 78.4) (end 149.2 80.4125) (width 0.35) (layer "F.Cu") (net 9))
 (segment (start 149.2875 82.4875) (end 150.8 84) (width 0.35) (layer "F.Cu") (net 9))
 (via (at 152.3 84) (size 1) (drill 0.5) (layers "F.Cu" "B.Cu") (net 9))
 (segment (start 153.42 86.76) (end 153.42 85.12) (width 0.35) (layer "B.Cu") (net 9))
 (segment (start 153.42 85.12) (end 152.3 84) (width 0.35) (layer "B.Cu") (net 9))
 (segment (start 153.15 78.4) (end 153.15 80.4625) (width 0.35) (layer "F.Cu") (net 3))
 (segment (start 153.1875 82.4875) (end 154.6 83.9) (width 0.35) (layer "F.Cu") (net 3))
 (segment (start 153.15 80.4625) (end 153.1875 80.5) (width 0.35) (layer "F.Cu") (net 3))
 (segment (start 153.1875 80.5) (end 153.1875 82.4875) (width 0.35) (layer "F.Cu") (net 3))
 (via (at 154.6 83.9) (size 1) (drill 0.5) (layers "F.Cu" "B.Cu") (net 3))
 (segment (start 155.96 86.76) (end 155.96 85.26) (width 0.35) (layer "B.Cu") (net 3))
 (segment (start 155.96 85.26) (end 154.6 83.9) (width 0.35) (layer "B.Cu") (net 3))
 (segment (start 166.3 76.8) (end 166.3 81.7) (width 0.35) (layer "F.Cu") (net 8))
 (segment (start 164.9 75.4) (end 165.7 76.2) (width 0.35) (layer "F.Cu") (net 8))
 (segment (start 163.9 75.4) (end 164.9 75.4) (width 0.35) (layer "F.Cu") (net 8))
 (segment (start 166.3 81.7) (end 166.3 81.9) (width 0.35) (layer "F.Cu") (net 8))
 (segment (start 165.7 76.2) (end 166.3 76.8) (width 0.35) (layer "F.Cu") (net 8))
 (via (at 166.3 81.9) (size 1) (drill 0.5) (layers "F.Cu" "B.Cu") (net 8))
 (segment (start 168.66 84.26) (end 168.66 86.76) (width 0.35) (layer "B.Cu") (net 8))
 (segment (start 166.3 81.9) (end 168.66 84.26) (width 0.35) (layer "B.Cu") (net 8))
 (segment (start 158.35 78.4) (end 156.7 78.4) (width 0.35) (layer "F.Cu") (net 1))
 (segment (start 158.4375 80.5) (end 158.4375 82.2625) (width 0.35) (layer "F.Cu") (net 1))
 (segment (start 154.2 96.9) (end 169.2 96.9) (width 0.35) (layer "F.Cu") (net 1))
 (segment (start 158.35 78.4) (end 158.35 80.4125) (width 0.35) (layer "F.Cu") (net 1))
 (segment (start 158.35 80.4125) (end 158.4375 80.5) (width 0.35) (layer "F.Cu") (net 1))
 (segment (start 152.4 96.9) (end 154.2 96.9) (width 0.35) (layer "F.Cu") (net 1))
 (segment (start 158.4375 82.2625) (end 149.95 90.75) (width 0.35) (layer "F.Cu") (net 1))
 (segment (start 149.95 90.75) (end 149.95 94.45) (width 0.35) (layer "F.Cu") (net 1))
 (segment (start 149.95 94.45) (end 152.4 96.9) (width 0.35) (layer "F.Cu") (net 1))
 (via (at 156.7 78.4) (size 1) (drill 0.5) (layers "F.Cu" "B.Cu") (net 1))
 (segment (start 156.7 78.4) (end 150.65 72.35) (width 0.35) (layer "B.Cu") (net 1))
 (segment (start 150.65 72.35) (end 150.65 69.25) (width 0.35) (layer "B.Cu") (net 1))
 (segment (start 157.8 75.4) (end 159.3 75.4) (width 0.35) (layer "F.Cu") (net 6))
 (segment (start 159.9 75.4) (end 162.9 78.4) (width 0.35) (layer "F.Cu") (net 6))
 (segment (start 152.5 76.9) (end 156.3 76.9) (width 0.35) (layer "F.Cu") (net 6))
 (segment (start 162.95 80.4625) (end 162.9875 80.5) (width 0.35) (layer "F.Cu") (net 6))
 (segment (start 162.95 78.4) (end 162.95 80.4625) (width 0.35) (layer "F.Cu") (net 6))
 (segment (start 162.9 78.4) (end 162.95 78.4) (width 0.35) (layer "F.Cu") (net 6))
 (segment (start 150.15 75.4) (end 151 75.4) (width 0.35) (layer "F.Cu") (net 6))
 (segment (start 156.3 76.9) (end 157.8 75.4) (width 0.35) (layer "F.Cu") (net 6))
 (segment (start 151 75.4) (end 152.5 76.9) (width 0.35) (layer "F.Cu") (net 6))
 (segment (start 159.3 75.4) (end 159.9 75.4) (width 0.35) (layer "F.Cu") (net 6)))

